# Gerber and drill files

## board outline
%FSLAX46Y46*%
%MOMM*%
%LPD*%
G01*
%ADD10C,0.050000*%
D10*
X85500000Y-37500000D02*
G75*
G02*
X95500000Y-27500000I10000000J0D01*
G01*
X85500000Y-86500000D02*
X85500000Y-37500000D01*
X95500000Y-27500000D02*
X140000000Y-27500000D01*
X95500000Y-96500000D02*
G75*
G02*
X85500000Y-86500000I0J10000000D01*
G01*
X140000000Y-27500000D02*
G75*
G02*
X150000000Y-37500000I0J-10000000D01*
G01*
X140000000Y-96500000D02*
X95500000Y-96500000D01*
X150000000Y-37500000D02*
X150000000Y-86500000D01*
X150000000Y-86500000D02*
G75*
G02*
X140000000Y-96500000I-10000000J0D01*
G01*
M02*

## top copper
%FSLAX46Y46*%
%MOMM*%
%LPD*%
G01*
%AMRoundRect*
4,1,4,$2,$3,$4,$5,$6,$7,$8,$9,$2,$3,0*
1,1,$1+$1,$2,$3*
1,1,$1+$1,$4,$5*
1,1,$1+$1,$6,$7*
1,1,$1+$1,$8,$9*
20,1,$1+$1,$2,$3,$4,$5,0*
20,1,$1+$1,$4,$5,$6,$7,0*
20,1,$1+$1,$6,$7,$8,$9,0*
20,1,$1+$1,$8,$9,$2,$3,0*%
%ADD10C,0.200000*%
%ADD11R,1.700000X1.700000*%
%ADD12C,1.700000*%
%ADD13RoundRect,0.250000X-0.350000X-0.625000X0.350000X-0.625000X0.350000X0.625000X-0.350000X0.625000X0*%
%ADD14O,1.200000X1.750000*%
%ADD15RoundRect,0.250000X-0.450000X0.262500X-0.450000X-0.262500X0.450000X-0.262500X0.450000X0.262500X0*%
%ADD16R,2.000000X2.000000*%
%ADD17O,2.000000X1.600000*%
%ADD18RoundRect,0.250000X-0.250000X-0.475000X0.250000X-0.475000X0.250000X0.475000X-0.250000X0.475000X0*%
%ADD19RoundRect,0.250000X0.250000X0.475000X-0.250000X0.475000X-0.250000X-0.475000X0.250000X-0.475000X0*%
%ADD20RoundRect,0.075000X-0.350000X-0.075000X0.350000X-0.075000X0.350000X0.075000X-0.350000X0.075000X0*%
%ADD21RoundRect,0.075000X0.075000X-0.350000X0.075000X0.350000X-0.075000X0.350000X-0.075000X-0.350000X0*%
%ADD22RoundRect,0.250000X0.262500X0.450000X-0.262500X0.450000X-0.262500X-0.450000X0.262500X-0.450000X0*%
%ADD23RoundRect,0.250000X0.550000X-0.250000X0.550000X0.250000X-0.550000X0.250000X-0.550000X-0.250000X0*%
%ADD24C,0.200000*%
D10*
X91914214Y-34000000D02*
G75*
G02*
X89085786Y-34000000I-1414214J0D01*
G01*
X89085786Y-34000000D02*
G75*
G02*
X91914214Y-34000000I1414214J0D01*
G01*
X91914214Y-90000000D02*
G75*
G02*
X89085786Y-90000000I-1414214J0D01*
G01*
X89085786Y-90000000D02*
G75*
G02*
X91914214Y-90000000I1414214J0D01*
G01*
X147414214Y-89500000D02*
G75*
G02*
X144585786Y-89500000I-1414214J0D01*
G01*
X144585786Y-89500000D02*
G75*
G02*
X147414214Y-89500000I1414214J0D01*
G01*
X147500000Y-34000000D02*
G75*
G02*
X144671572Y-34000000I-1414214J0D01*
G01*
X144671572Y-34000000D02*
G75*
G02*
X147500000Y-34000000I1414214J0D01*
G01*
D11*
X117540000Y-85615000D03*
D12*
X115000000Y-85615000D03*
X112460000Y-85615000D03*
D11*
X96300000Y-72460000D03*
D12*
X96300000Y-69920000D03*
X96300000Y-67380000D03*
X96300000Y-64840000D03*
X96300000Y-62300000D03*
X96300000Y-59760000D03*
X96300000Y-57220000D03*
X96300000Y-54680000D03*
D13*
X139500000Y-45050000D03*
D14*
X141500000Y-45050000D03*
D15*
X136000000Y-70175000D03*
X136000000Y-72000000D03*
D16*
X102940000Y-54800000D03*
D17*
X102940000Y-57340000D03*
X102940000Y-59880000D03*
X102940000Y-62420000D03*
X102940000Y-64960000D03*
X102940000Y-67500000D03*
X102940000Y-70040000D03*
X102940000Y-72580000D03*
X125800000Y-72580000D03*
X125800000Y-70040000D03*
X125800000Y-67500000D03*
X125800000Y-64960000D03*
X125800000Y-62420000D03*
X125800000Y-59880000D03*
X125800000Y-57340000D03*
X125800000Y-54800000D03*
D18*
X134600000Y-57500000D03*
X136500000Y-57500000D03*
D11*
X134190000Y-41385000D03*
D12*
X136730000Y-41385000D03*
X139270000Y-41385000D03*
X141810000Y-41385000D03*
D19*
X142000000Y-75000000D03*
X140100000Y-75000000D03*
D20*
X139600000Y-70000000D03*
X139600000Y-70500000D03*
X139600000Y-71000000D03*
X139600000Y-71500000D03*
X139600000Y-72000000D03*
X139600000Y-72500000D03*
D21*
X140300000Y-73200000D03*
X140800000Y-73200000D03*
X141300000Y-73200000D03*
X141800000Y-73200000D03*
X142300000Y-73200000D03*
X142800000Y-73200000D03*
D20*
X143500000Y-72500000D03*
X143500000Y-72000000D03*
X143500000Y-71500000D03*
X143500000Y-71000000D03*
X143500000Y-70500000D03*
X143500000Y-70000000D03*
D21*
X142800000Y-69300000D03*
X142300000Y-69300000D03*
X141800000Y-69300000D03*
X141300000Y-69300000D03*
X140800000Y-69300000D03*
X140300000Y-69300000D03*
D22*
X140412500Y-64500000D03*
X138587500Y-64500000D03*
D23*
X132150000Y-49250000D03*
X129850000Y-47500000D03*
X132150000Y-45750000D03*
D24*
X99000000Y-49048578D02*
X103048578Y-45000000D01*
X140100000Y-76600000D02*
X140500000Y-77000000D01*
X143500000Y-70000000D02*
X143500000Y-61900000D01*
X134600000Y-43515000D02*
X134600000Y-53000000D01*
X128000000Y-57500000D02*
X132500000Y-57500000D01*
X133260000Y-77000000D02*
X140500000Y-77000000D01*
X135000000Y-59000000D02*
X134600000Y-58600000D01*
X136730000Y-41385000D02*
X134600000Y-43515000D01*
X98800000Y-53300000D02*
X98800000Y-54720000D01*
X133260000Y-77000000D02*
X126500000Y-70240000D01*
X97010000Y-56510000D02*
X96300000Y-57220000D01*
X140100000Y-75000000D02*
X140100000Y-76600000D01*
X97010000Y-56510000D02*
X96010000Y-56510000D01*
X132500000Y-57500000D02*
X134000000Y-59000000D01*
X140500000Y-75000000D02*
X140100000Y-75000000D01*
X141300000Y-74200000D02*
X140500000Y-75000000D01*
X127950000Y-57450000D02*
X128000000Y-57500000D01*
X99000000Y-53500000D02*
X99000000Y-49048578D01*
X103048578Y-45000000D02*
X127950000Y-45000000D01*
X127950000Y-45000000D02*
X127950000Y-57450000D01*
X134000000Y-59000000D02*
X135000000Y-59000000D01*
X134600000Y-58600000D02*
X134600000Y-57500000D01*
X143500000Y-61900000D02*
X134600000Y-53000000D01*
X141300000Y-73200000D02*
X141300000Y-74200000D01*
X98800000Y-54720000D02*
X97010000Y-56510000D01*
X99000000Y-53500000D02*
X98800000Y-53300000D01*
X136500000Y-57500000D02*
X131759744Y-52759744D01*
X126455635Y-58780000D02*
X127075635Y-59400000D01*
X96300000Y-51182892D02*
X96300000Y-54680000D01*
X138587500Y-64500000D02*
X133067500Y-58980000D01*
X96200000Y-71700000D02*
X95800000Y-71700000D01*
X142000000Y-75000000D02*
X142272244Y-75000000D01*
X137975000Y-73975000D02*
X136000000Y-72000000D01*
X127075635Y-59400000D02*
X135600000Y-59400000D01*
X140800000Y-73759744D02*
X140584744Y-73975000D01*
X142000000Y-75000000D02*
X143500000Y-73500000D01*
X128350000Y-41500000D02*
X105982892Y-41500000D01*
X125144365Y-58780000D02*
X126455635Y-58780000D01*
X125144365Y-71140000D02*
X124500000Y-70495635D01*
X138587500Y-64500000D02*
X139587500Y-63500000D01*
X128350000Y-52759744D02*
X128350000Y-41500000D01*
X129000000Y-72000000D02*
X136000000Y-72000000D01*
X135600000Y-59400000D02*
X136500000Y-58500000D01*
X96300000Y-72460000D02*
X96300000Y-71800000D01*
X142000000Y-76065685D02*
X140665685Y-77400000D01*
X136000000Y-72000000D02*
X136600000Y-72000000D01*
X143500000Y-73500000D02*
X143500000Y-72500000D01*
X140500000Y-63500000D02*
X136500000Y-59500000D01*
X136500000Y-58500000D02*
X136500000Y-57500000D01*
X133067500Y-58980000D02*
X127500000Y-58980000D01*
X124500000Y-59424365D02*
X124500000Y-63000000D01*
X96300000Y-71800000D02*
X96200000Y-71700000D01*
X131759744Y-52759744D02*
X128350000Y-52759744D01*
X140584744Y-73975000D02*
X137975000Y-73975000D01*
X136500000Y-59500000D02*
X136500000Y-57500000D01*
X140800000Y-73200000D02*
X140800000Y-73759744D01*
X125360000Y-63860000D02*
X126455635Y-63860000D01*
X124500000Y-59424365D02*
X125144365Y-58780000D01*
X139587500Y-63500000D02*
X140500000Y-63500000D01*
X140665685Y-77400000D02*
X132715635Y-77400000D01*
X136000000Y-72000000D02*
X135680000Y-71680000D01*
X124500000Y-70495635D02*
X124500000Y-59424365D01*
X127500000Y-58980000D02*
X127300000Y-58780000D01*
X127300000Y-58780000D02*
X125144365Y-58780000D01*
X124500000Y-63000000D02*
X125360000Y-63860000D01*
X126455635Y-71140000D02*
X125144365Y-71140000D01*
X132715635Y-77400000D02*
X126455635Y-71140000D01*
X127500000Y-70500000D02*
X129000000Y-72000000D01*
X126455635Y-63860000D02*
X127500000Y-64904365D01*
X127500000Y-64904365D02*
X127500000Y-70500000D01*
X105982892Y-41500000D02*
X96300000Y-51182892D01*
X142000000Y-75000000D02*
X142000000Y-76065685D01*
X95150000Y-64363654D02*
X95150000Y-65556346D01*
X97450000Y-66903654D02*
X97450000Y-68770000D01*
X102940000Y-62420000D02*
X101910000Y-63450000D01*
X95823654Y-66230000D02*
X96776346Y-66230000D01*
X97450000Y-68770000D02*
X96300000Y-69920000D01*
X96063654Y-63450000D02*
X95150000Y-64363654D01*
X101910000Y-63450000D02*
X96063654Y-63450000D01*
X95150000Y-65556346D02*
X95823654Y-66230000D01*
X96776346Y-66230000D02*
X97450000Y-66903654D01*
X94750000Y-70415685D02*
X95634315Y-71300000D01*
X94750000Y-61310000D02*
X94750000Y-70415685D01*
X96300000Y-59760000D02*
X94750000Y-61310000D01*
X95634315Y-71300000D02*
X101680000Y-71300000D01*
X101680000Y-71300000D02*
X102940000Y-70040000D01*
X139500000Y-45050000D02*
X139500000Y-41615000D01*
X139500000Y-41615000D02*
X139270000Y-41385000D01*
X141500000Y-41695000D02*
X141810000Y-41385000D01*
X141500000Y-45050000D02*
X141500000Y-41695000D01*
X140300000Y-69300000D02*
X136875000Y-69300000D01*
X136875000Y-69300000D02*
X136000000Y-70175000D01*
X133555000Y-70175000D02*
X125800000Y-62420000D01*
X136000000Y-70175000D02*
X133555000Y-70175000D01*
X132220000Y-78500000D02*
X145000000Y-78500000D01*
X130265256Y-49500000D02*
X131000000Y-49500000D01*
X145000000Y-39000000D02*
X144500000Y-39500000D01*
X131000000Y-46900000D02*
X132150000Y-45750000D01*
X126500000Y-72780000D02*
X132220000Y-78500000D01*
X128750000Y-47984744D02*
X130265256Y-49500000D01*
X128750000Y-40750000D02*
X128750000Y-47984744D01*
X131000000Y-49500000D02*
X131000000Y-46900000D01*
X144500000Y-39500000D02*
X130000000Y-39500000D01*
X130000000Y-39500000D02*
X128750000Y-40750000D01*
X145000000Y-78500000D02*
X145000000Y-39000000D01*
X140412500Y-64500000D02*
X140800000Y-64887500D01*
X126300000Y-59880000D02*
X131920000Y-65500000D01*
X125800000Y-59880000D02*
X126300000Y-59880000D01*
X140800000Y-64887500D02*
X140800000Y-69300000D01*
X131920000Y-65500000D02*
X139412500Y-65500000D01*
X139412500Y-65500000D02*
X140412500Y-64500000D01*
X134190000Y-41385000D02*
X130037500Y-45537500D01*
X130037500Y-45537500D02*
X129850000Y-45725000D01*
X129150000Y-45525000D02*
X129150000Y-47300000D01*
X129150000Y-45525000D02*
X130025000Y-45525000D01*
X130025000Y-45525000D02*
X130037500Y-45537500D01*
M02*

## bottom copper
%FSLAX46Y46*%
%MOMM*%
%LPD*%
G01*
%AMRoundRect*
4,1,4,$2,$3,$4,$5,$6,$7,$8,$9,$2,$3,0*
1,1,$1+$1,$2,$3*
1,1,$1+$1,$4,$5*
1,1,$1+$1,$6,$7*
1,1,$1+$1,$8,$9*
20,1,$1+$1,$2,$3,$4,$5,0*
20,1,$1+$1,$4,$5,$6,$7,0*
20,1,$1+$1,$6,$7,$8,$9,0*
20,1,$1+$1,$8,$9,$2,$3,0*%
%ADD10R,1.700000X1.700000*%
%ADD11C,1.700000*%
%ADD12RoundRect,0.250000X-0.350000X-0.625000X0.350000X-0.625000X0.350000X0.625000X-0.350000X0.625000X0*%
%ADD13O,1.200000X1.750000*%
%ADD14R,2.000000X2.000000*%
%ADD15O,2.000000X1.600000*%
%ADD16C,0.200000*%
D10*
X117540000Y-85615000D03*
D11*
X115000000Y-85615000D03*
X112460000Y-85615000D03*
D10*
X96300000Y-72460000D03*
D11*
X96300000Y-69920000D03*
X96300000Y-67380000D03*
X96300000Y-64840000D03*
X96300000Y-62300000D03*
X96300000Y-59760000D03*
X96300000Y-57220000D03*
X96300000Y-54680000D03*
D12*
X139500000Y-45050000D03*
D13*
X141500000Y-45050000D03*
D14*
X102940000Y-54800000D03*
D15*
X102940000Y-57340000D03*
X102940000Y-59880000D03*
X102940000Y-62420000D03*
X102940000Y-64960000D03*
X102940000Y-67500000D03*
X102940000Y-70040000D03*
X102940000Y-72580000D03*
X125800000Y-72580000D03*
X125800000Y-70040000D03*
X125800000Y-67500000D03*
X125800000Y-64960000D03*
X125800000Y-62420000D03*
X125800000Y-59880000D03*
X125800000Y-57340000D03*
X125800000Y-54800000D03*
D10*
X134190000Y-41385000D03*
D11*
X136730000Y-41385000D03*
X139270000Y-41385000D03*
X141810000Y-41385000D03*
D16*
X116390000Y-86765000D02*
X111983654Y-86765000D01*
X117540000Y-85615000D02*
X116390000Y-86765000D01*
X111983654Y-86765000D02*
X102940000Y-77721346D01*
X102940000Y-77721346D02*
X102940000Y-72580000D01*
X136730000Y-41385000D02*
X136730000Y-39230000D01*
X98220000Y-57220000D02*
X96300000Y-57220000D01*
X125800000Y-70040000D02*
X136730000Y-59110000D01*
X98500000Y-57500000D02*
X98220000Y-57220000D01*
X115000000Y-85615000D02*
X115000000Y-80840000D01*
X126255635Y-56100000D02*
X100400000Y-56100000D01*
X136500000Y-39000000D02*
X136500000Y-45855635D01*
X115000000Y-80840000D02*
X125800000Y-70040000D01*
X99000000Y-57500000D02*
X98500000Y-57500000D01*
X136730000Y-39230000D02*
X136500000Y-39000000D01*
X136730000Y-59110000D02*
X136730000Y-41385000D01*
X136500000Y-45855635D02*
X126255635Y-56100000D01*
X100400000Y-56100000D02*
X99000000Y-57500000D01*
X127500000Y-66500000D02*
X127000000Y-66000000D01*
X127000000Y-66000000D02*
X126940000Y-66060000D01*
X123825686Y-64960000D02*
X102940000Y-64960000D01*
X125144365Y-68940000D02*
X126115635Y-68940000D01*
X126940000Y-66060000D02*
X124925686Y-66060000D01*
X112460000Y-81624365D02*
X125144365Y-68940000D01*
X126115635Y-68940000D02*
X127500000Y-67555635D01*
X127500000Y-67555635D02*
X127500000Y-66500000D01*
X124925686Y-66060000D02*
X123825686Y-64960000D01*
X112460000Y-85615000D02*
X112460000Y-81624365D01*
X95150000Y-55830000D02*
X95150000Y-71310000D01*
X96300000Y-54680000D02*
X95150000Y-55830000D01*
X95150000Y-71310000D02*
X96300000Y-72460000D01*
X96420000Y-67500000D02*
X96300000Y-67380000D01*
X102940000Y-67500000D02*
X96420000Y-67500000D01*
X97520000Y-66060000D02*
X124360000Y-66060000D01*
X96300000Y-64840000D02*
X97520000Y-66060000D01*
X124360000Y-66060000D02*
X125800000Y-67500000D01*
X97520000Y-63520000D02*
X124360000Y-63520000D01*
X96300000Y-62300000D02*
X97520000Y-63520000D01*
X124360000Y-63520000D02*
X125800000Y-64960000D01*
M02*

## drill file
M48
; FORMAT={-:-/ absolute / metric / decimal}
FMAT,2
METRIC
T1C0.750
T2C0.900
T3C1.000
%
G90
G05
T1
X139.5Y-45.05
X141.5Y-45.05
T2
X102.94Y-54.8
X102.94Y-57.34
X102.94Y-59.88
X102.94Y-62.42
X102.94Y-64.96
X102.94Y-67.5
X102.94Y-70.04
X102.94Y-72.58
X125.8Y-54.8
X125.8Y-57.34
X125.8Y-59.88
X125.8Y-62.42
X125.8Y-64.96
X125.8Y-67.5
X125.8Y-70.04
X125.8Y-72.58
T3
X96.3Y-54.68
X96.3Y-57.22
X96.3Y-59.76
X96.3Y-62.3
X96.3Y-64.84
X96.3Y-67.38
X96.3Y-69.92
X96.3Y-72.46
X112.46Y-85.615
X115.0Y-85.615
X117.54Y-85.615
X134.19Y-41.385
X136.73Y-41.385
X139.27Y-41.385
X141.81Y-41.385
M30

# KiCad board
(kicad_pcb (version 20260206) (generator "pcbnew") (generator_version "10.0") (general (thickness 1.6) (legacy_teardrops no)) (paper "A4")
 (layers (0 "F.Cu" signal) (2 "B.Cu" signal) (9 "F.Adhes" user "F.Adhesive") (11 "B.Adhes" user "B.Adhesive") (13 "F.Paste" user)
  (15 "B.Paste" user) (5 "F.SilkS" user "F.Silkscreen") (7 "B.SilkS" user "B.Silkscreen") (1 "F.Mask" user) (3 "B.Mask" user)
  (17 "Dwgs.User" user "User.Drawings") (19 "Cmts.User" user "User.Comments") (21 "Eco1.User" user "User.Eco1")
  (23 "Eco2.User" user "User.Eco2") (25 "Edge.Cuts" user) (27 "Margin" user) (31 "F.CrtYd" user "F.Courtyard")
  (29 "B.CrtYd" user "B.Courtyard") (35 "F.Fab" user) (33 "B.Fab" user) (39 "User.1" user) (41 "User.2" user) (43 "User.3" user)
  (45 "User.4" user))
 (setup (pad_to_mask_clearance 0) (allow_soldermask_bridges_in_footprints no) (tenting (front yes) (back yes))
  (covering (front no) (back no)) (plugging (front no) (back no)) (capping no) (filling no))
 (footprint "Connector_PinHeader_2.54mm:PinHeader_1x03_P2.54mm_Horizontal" (layer "F.Cu") (at 117.54 85.615 -90)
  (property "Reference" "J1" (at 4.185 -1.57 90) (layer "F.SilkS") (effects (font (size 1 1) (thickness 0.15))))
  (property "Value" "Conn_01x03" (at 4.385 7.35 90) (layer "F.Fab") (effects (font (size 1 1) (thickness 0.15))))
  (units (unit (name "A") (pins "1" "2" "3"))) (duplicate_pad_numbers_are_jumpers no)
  (pad "1" thru_hole rect (at 0 0 270) (size 1.7 1.7) (drill 1) (layers "*.Cu" "*.Mask") (remove_unused_layers no) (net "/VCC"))
  (pad "2" thru_hole circle (at 0 2.54 270) (size 1.7 1.7) (drill 1) (layers "*.Cu" "*.Mask") (remove_unused_layers no) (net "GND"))
  (pad "3" thru_hole circle (at 0 5.08 270) (size 1.7 1.7) (drill 1) (layers "*.Cu" "*.Mask") (remove_unused_layers no) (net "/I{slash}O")))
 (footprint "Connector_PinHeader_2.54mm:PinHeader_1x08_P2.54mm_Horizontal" (layer "F.Cu") (at 96.3 72.46 180)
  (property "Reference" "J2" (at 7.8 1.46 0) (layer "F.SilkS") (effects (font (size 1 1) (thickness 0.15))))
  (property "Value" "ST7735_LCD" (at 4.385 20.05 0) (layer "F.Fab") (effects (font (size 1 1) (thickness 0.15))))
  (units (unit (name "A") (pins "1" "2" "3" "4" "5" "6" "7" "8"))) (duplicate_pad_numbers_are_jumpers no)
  (pad "1" thru_hole rect (at 0 0 180) (size 1.7 1.7) (drill 1) (layers "*.Cu" "*.Mask") (remove_unused_layers no) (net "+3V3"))
  (pad "2" thru_hole circle (at 0 2.54 180) (size 1.7 1.7) (drill 1) (layers "*.Cu" "*.Mask") (remove_unused_layers no) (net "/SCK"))
  (pad "3" thru_hole circle (at 0 5.08 180) (size 1.7 1.7) (drill 1) (layers "*.Cu" "*.Mask") (remove_unused_layers no) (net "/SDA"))
  (pad "4" thru_hole circle (at 0 7.62 180) (size 1.7 1.7) (drill 1) (layers "*.Cu" "*.Mask") (remove_unused_layers no) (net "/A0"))
  (pad "5" thru_hole circle (at 0 10.16 180) (size 1.7 1.7) (drill 1) (layers "*.Cu" "*.Mask") (remove_unused_layers no) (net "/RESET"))
  (pad "6" thru_hole circle (at 0 12.7 180) (size 1.7 1.7) (drill 1) (layers "*.Cu" "*.Mask") (remove_unused_layers no) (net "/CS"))
  (pad "7" thru_hole circle (at 0 15.24 180) (size 1.7 1.7) (drill 1) (layers "*.Cu" "*.Mask") (remove_unused_layers no) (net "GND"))
  (pad "8" thru_hole circle (at 0 17.78 180) (size 1.7 1.7) (drill 1) (layers "*.Cu" "*.Mask") (remove_unused_layers no) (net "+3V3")))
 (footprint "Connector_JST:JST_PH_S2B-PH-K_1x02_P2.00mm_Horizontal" (layer "F.Cu") (at 139.5 45.05)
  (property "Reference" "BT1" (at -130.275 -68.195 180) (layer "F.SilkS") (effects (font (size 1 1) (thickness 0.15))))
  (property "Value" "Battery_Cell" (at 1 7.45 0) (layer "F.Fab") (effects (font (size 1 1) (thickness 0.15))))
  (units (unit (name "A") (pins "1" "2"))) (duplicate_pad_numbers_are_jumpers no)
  (pad "1" thru_hole roundrect (at 0 0) (size 1.2 1.75) (drill 0.75) (layers "*.Cu" "*.Mask") (remove_unused_layers no)
   (roundrect_rratio 0.208333) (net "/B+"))
  (pad "2" thru_hole oval (at 2 0) (size 1.2 1.75) (drill 0.75) (layers "*.Cu" "*.Mask") (remove_unused_layers no) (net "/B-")))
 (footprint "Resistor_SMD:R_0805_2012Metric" (layer "F.Cu") (at 136 71.0875 -90)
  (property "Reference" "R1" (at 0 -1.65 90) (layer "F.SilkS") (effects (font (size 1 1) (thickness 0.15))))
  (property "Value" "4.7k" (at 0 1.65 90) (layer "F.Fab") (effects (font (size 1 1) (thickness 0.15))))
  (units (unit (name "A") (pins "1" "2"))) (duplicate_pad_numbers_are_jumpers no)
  (pad "1" smd roundrect (at -0.9125 0 270) (size 1.025 1.4) (layers "F.Cu" "F.Mask" "F.Paste") (roundrect_rratio 0.243902)
   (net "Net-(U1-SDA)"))
  (pad "2" smd roundrect (at 0.9125 0 270) (size 1.025 1.4) (layers "F.Cu" "F.Mask" "F.Paste") (roundrect_rratio 0.243902) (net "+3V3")))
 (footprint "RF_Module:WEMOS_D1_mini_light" (layer "F.Cu") (at 102.94 54.8)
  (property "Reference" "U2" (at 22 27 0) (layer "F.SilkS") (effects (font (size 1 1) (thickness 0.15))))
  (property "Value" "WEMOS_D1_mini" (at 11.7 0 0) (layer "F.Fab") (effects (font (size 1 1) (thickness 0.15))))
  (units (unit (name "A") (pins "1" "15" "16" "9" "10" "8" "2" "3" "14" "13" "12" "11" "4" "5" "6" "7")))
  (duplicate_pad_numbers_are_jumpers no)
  (pad "1" thru_hole rect (at 0 0) (size 2 2) (drill 0.9) (layers "*.Cu" "*.Mask") (remove_unused_layers no)
   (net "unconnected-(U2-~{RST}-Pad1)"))
  (pad "2" thru_hole oval (at 0 2.54) (size 2 1.6) (drill 0.9) (layers "*.Cu" "*.Mask") (remove_unused_layers no)
   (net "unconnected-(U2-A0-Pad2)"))
  (pad "3" thru_hole oval (at 0 5.08) (size 2 1.6) (drill 0.9) (layers "*.Cu" "*.Mask") (remove_unused_layers no)
   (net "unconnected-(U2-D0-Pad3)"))
  (pad "4" thru_hole oval (at 0 7.62) (size 2 1.6) (drill 0.9) (layers "*.Cu" "*.Mask") (remove_unused_layers no) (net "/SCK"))
  (pad "5" thru_hole oval (at 0 10.16) (size 2 1.6) (drill 0.9) (layers "*.Cu" "*.Mask") (remove_unused_layers no) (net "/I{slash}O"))
  (pad "6" thru_hole oval (at 0 12.7) (size 2 1.6) (drill 0.9) (layers "*.Cu" "*.Mask") (remove_unused_layers no) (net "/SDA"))
  (pad "7" thru_hole oval (at 0 15.24) (size 2 1.6) (drill 0.9) (layers "*.Cu" "*.Mask") (remove_unused_layers no) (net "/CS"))
  (pad "8" thru_hole oval (at 0 17.78) (size 2 1.6) (drill 0.9) (layers "*.Cu" "*.Mask") (remove_unused_layers no) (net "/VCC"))
  (pad "9" thru_hole oval (at 22.86 17.78) (size 2 1.6) (drill 0.9) (layers "*.Cu" "*.Mask") (remove_unused_layers no) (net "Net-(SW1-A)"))
  (pad "10" thru_hole oval (at 22.86 15.24) (size 2 1.6) (drill 0.9) (layers "*.Cu" "*.Mask") (remove_unused_layers no) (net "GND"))
  (pad "11" thru_hole oval (at 22.86 12.7) (size 2 1.6) (drill 0.9) (layers "*.Cu" "*.Mask") (remove_unused_layers no) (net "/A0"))
  (pad "12" thru_hole oval (at 22.86 10.16) (size 2 1.6) (drill 0.9) (layers "*.Cu" "*.Mask") (remove_unused_layers no) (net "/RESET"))
  (pad "13" thru_hole oval (at 22.86 7.62) (size 2 1.6) (drill 0.9) (layers "*.Cu" "*.Mask") (remove_unused_layers no) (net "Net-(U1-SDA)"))
  (pad "14" thru_hole oval (at 22.86 5.08) (size 2 1.6) (drill 0.9) (layers "*.Cu" "*.Mask") (remove_unused_layers no) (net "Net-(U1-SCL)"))
  (pad "15" thru_hole oval (at 22.86 2.54) (size 2 1.6) (drill 0.9) (layers "*.Cu" "*.Mask") (remove_unused_layers no)
   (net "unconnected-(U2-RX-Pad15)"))
  (pad "16" thru_hole oval (at 22.86 0) (size 2 1.6) (drill 0.9) (layers "*.Cu" "*.Mask") (remove_unused_layers no)
   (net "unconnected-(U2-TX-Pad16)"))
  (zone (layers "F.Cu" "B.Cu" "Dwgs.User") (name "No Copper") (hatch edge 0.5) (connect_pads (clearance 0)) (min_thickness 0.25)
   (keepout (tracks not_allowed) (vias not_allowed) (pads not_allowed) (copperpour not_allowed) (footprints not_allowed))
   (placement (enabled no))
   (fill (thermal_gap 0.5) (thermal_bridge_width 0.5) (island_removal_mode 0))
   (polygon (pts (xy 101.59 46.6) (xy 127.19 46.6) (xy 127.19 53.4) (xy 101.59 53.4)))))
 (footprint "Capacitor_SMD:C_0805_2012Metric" (layer "F.Cu") (at 135.55 57.5)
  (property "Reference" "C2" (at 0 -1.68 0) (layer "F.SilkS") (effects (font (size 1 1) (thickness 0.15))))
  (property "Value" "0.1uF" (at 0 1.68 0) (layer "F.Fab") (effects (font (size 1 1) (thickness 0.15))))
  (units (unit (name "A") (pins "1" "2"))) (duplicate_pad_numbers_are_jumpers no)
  (pad "1" smd roundrect (at -0.95 0) (size 1 1.45) (layers "F.Cu" "F.Mask" "F.Paste") (roundrect_rratio 0.25) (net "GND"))
  (pad "2" smd roundrect (at 0.95 0) (size 1 1.45) (layers "F.Cu" "F.Mask" "F.Paste") (roundrect_rratio 0.25) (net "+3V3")))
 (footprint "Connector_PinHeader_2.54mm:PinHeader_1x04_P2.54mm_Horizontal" (layer "F.Cu") (at 134.19 41.385 90)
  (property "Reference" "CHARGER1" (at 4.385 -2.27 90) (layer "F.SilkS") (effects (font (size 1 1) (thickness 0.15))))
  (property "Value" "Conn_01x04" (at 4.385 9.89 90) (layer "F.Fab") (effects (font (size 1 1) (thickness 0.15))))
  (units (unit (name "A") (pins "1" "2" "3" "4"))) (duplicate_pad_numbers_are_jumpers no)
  (pad "1" thru_hole rect (at 0 0 90) (size 1.7 1.7) (drill 1) (layers "*.Cu" "*.Mask") (remove_unused_layers no) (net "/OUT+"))
  (pad "2" thru_hole circle (at 0 2.54 90) (size 1.7 1.7) (drill 1) (layers "*.Cu" "*.Mask") (remove_unused_layers no) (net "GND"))
  (pad "3" thru_hole circle (at 0 5.08 90) (size 1.7 1.7) (drill 1) (layers "*.Cu" "*.Mask") (remove_unused_layers no) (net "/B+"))
  (pad "4" thru_hole circle (at 0 7.62 90) (size 1.7 1.7) (drill 1) (layers "*.Cu" "*.Mask") (remove_unused_layers no) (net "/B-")))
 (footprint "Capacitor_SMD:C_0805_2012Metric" (layer "F.Cu") (at 141.05 75 180)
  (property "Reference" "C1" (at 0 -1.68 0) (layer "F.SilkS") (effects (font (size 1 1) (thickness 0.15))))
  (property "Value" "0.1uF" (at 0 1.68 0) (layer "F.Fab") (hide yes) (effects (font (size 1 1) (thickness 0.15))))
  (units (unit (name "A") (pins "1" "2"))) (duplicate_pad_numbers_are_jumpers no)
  (pad "1" smd roundrect (at -0.95 0 180) (size 1 1.45) (layers "F.Cu" "F.Mask" "F.Paste") (roundrect_rratio 0.25) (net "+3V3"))
  (pad "2" smd roundrect (at 0.95 0 180) (size 1 1.45) (layers "F.Cu" "F.Mask" "F.Paste") (roundrect_rratio 0.25) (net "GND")))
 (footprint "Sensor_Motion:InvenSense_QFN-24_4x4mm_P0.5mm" (layer "F.Cu") (at 141.55 71.25)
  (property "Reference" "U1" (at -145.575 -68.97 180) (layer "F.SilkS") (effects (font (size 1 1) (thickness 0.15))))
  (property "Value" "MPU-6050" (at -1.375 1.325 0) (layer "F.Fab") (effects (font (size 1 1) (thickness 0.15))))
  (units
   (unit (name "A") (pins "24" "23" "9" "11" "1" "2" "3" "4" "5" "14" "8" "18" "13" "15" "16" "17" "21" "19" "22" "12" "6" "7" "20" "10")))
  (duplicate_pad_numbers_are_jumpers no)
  (pad "1" smd roundrect (at -1.95 -1.25) (size 0.85 0.3) (layers "F.Cu" "F.Mask" "F.Paste") (roundrect_rratio 0.25)
   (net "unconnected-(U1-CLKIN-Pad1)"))
  (pad "2" smd roundrect (at -1.95 -0.75) (size 0.85 0.3) (layers "F.Cu" "F.Mask" "F.Paste") (roundrect_rratio 0.25)
   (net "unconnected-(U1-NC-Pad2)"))
  (pad "3" smd roundrect (at -1.95 -0.25) (size 0.85 0.3) (layers "F.Cu" "F.Mask" "F.Paste") (roundrect_rratio 0.25)
   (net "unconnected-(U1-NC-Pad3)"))
  (pad "4" smd roundrect (at -1.95 0.25) (size 0.85 0.3) (layers "F.Cu" "F.Mask" "F.Paste") (roundrect_rratio 0.25)
   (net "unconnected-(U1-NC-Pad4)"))
  (pad "5" smd roundrect (at -1.95 0.75) (size 0.85 0.3) (layers "F.Cu" "F.Mask" "F.Paste") (roundrect_rratio 0.25)
   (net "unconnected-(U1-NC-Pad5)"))
  (pad "6" smd roundrect (at -1.95 1.25) (size 0.85 0.3) (layers "F.Cu" "F.Mask" "F.Paste") (roundrect_rratio 0.25)
   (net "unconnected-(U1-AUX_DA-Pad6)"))
  (pad "7" smd roundrect (at -1.25 1.95 90) (size 0.85 0.3) (layers "F.Cu" "F.Mask" "F.Paste") (roundrect_rratio 0.25)
   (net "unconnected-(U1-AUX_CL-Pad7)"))
  (pad "8" smd roundrect (at -0.75 1.95 90) (size 0.85 0.3) (layers "F.Cu" "F.Mask" "F.Paste") (roundrect_rratio 0.25) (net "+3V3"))
  (pad "9" smd roundrect (at -0.25 1.95 90) (size 0.85 0.3) (layers "F.Cu" "F.Mask" "F.Paste") (roundrect_rratio 0.25) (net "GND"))
  (pad "10" smd roundrect (at 0.25 1.95 90) (size 0.85 0.3) (layers "F.Cu" "F.Mask" "F.Paste") (roundrect_rratio 0.25)
   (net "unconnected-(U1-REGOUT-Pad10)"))
  (pad "11" smd roundrect (at 0.75 1.95 90) (size 0.85 0.3) (layers "F.Cu" "F.Mask" "F.Paste") (roundrect_rratio 0.25)
   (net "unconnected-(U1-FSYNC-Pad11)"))
  (pad "12" smd roundrect (at 1.25 1.95 90) (size 0.85 0.3) (layers "F.Cu" "F.Mask" "F.Paste") (roundrect_rratio 0.25)
   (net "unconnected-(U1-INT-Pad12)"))
  (pad "13" smd roundrect (at 1.95 1.25) (size 0.85 0.3) (layers "F.Cu" "F.Mask" "F.Paste") (roundrect_rratio 0.25) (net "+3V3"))
  (pad "14" smd roundrect (at 1.95 0.75) (size 0.85 0.3) (layers "F.Cu" "F.Mask" "F.Paste") (roundrect_rratio 0.25)
   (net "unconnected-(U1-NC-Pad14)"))
  (pad "15" smd roundrect (at 1.95 0.25) (size 0.85 0.3) (layers "F.Cu" "F.Mask" "F.Paste") (roundrect_rratio 0.25)
   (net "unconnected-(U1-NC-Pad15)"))
  (pad "16" smd roundrect (at 1.95 -0.25) (size 0.85 0.3) (layers "F.Cu" "F.Mask" "F.Paste") (roundrect_rratio 0.25)
   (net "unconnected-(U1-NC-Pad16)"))
  (pad "17" smd roundrect (at 1.95 -0.75) (size 0.85 0.3) (layers "F.Cu" "F.Mask" "F.Paste") (roundrect_rratio 0.25)
   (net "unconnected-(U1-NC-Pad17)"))
  (pad "18" smd roundrect (at 1.95 -1.25) (size 0.85 0.3) (layers "F.Cu" "F.Mask" "F.Paste") (roundrect_rratio 0.25) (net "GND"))
  (pad "19" smd roundrect (at 1.25 -1.95 90) (size 0.85 0.3) (layers "F.Cu" "F.Mask" "F.Paste") (roundrect_rratio 0.25)
   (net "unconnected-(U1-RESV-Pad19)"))
  (pad "20" smd roundrect (at 0.75 -1.95 90) (size 0.85 0.3) (layers "F.Cu" "F.Mask" "F.Paste") (roundrect_rratio 0.25)
   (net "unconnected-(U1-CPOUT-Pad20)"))
  (pad "21" smd roundrect (at 0.25 -1.95 90) (size 0.85 0.3) (layers "F.Cu" "F.Mask" "F.Paste") (roundrect_rratio 0.25)
   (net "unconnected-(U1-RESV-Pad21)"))
  (pad "22" smd roundrect (at -0.25 -1.95 90) (size 0.85 0.3) (layers "F.Cu" "F.Mask" "F.Paste") (roundrect_rratio 0.25)
   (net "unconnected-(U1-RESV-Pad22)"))
  (pad "23" smd roundrect (at -0.75 -1.95 90) (size 0.85 0.3) (layers "F.Cu" "F.Mask" "F.Paste") (roundrect_rratio 0.25)
   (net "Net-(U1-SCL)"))
  (pad "24" smd roundrect (at -1.25 -1.95 90) (size 0.85 0.3) (layers "F.Cu" "F.Mask" "F.Paste") (roundrect_rratio 0.25)
   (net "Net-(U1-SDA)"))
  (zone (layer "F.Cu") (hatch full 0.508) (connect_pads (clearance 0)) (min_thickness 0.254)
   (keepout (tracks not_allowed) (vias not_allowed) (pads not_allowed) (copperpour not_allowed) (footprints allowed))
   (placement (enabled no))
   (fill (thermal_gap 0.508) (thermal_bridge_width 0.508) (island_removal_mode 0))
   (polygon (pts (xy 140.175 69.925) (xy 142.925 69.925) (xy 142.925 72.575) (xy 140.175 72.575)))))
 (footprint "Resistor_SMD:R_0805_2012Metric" (layer "F.Cu") (at 139.5 64.5 180)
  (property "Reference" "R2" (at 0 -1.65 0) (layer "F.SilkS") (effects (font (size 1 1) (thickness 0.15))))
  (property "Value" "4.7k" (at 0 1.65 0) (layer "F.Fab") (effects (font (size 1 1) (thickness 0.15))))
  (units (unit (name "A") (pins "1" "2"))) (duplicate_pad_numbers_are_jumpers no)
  (pad "1" smd roundrect (at -0.9125 0 180) (size 1.025 1.4) (layers "F.Cu" "F.Mask" "F.Paste") (roundrect_rratio 0.243902)
   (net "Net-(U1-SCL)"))
  (pad "2" smd roundrect (at 0.9125 0 180) (size 1.025 1.4) (layers "F.Cu" "F.Mask" "F.Paste") (roundrect_rratio 0.243902) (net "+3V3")))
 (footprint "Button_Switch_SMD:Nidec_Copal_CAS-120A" (layer "F.Cu") (at 131 47.5 180)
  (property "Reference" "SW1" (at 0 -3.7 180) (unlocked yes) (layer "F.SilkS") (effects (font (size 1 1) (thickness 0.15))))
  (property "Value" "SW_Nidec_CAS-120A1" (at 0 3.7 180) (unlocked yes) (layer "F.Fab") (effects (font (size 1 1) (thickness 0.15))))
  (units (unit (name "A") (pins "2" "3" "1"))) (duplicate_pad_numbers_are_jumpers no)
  (pad "1" smd roundrect (at -1.15 -1.75 90) (size 1 1.6) (layers "F.Cu" "F.Mask" "F.Paste") (roundrect_rratio 0.25)
   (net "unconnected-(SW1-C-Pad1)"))
  (pad "2" smd roundrect (at 1.15 0 90) (size 1 1.6) (layers "F.Cu" "F.Mask" "F.Paste") (roundrect_rratio 0.25) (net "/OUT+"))
  (pad "3" smd roundrect (at -1.15 1.75 90) (size 1 1.6) (layers "F.Cu" "F.Mask" "F.Paste") (roundrect_rratio 0.25) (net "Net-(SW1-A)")))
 (gr_circle (center 90.5 34) (end 91.5 35) (stroke (width 0.2) (type default)) (fill no) (layer "F.Cu"))
 (gr_circle (center 90.5 90) (end 91.5 91) (stroke (width 0.2) (type default)) (fill no) (layer "F.Cu"))
 (gr_circle (center 146 89.5) (end 147 90.5) (stroke (width 0.2) (type default)) (fill no) (layer "F.Cu"))
 (gr_circle (center 146.085786 34) (end 147.085786 35) (stroke (width 0.2) (type default)) (fill no) (layer "F.Cu"))
 (gr_arc (start 85.5 37.5) (mid 88.428932 30.428932) (end 95.5 27.5) (stroke (width 0.05) (type default)) (layer "Edge.Cuts"))
 (gr_line (start 85.5 86.5) (end 85.5 37.5) (stroke (width 0.05) (type default)) (layer "Edge.Cuts"))
 (gr_line (start 95.5 27.5) (end 140 27.5) (stroke (width 0.05) (type default)) (layer "Edge.Cuts"))
 (gr_arc (start 95.5 96.5) (mid 88.428932 93.571068) (end 85.5 86.5) (stroke (width 0.05) (type default)) (layer "Edge.Cuts"))
 (gr_arc (start 140 27.5) (mid 147.071068 30.428932) (end 150 37.5) (stroke (width 0.05) (type default)) (layer "Edge.Cuts"))
 (gr_line (start 140 96.5) (end 95.5 96.5) (stroke (width 0.05) (type default)) (layer "Edge.Cuts"))
 (gr_line (start 150 37.5) (end 150 86.5) (stroke (width 0.05) (type default)) (layer "Edge.Cuts"))
 (gr_arc (start 150 86.5) (mid 147.071068 93.571068) (end 140 96.5) (stroke (width 0.05) (type default)) (layer "Edge.Cuts"))
 (segment (start 116.39 86.765) (end 111.983654 86.765) (width 0.2) (layer "B.Cu") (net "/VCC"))
 (segment (start 117.54 85.615) (end 116.39 86.765) (width 0.2) (layer "B.Cu") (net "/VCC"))
 (segment (start 111.983654 86.765) (end 102.94 77.721346) (width 0.2) (layer "B.Cu") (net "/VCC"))
 (segment (start 102.94 77.721346) (end 102.94 72.58) (width 0.2) (layer "B.Cu") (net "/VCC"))
 (segment (start 99 49.048578) (end 103.048578 45) (width 0.2) (layer "F.Cu") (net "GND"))
 (segment (start 140.1 76.6) (end 140.5 77) (width 0.2) (layer "F.Cu") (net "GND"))
 (segment (start 143.5 70) (end 143.5 61.9) (width 0.2) (layer "F.Cu") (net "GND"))
 (segment (start 134.6 43.515) (end 134.6 53) (width 0.2) (layer "F.Cu") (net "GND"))
 (segment (start 128 57.5) (end 132.5 57.5) (width 0.2) (layer "F.Cu") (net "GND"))
 (segment (start 133.26 77) (end 140.5 77) (width 0.2) (layer "F.Cu") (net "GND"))
 (segment (start 135 59) (end 134.6 58.6) (width 0.2) (layer "F.Cu") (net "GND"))
 (segment (start 136.73 41.385) (end 134.6 43.515) (width 0.2) (layer "F.Cu") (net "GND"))
 (segment (start 98.8 53.3) (end 98.8 54.72) (width 0.2) (layer "F.Cu") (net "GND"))
 (segment (start 133.26 77) (end 126.5 70.24) (width 0.2) (layer "F.Cu") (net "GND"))
 (segment (start 97.01 56.51) (end 96.3 57.22) (width 0.2) (layer "F.Cu") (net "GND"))
 (segment (start 140.1 75) (end 140.1 76.6) (width 0.2) (layer "F.Cu") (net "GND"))
 (segment (start 97.01 56.51) (end 96.01 56.51) (width 0.2) (layer "F.Cu") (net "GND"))
 (segment (start 132.5 57.5) (end 134 59) (width 0.2) (layer "F.Cu") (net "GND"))
 (segment (start 140.5 75) (end 140.1 75) (width 0.2) (layer "F.Cu") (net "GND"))
 (segment (start 141.3 74.2) (end 140.5 75) (width 0.2) (layer "F.Cu") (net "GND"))
 (segment (start 127.95 57.45) (end 128 57.5) (width 0.2) (layer "F.Cu") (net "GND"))
 (segment (start 99 53.5) (end 99 49.048578) (width 0.2) (layer "F.Cu") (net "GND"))
 (segment (start 103.048578 45) (end 127.95 45) (width 0.2) (layer "F.Cu") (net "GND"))
 (segment (start 127.95 45) (end 127.95 57.45) (width 0.2) (layer "F.Cu") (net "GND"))
 (segment (start 134 59) (end 135 59) (width 0.2) (layer "F.Cu") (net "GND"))
 (segment (start 134.6 58.6) (end 134.6 57.5) (width 0.2) (layer "F.Cu") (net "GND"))
 (segment (start 143.5 61.9) (end 134.6 53) (width 0.2) (layer "F.Cu") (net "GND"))
 (segment (start 141.3 73.2) (end 141.3 74.2) (width 0.2) (layer "F.Cu") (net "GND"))
 (segment (start 98.8 54.72) (end 97.01 56.51) (width 0.2) (layer "F.Cu") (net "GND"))
 (segment (start 99 53.5) (end 98.8 53.3) (width 0.2) (layer "F.Cu") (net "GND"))
 (segment (start 136.73 41.385) (end 136.73 39.23) (width 0.2) (layer "B.Cu") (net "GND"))
 (segment (start 98.22 57.22) (end 96.3 57.22) (width 0.2) (layer "B.Cu") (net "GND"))
 (segment (start 125.8 70.04) (end 136.73 59.11) (width 0.2) (layer "B.Cu") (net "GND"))
 (segment (start 98.5 57.5) (end 98.22 57.22) (width 0.2) (layer "B.Cu") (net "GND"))
 (segment (start 115 85.615) (end 115 80.84) (width 0.2) (layer "B.Cu") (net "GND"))
 (segment (start 126.255635 56.1) (end 100.4 56.1) (width 0.2) (layer "B.Cu") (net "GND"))
 (segment (start 136.5 39) (end 136.5 45.855635) (width 0.2) (layer "B.Cu") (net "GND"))
 (segment (start 115 80.84) (end 125.8 70.04) (width 0.2) (layer "B.Cu") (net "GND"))
 (segment (start 99 57.5) (end 98.5 57.5) (width 0.2) (layer "B.Cu") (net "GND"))
 (segment (start 136.73 39.23) (end 136.5 39) (width 0.2) (layer "B.Cu") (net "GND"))
 (segment (start 136.73 59.11) (end 136.73 41.385) (width 0.2) (layer "B.Cu") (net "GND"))
 (segment (start 136.5 45.855635) (end 126.255635 56.1) (width 0.2) (layer "B.Cu") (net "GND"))
 (segment (start 100.4 56.1) (end 99 57.5) (width 0.2) (layer "B.Cu") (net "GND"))
 (segment (start 127.5 66.5) (end 127 66) (width 0.2) (layer "B.Cu") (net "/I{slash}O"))
 (segment (start 127 66) (end 126.94 66.06) (width 0.2) (layer "B.Cu") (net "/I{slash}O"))
 (segment (start 123.825686 64.96) (end 102.94 64.96) (width 0.2) (layer "B.Cu") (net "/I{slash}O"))
 (segment (start 125.144365 68.94) (end 126.115635 68.94) (width 0.2) (layer "B.Cu") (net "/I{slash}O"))
 (segment (start 126.94 66.06) (end 124.925686 66.06) (width 0.2) (layer "B.Cu") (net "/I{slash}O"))
 (segment (start 112.46 81.624365) (end 125.144365 68.94) (width 0.2) (layer "B.Cu") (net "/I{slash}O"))
 (segment (start 126.115635 68.94) (end 127.5 67.555635) (width 0.2) (layer "B.Cu") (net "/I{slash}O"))
 (segment (start 127.5 67.555635) (end 127.5 66.5) (width 0.2) (layer "B.Cu") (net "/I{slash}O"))
 (segment (start 124.925686 66.06) (end 123.825686 64.96) (width 0.2) (layer "B.Cu") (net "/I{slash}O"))
 (segment (start 112.46 85.615) (end 112.46 81.624365) (width 0.2) (layer "B.Cu") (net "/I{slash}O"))
 (segment (start 136.5 57.5) (end 131.759744 52.759744) (width 0.2) (layer "F.Cu") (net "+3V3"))
 (segment (start 126.455635 58.78) (end 127.075635 59.4) (width 0.2) (layer "F.Cu") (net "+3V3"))
 (segment (start 96.3 51.182892) (end 96.3 54.68) (width 0.2) (layer "F.Cu") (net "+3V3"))
 (segment (start 138.5875 64.5) (end 133.0675 58.98) (width 0.2) (layer "F.Cu") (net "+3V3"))
 (segment (start 96.2 71.7) (end 95.8 71.7) (width 0.2) (layer "F.Cu") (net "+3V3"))
 (segment (start 142 75) (end 142.272244 75) (width 0.2) (layer "F.Cu") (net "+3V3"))
 (segment (start 137.975 73.975) (end 136 72) (width 0.2) (layer "F.Cu") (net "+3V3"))
 (segment (start 127.075635 59.4) (end 135.6 59.4) (width 0.2) (layer "F.Cu") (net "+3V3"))
 (segment (start 140.8 73.759744) (end 140.584744 73.975) (width 0.2) (layer "F.Cu") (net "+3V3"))
 (segment (start 142 75) (end 143.5 73.5) (width 0.2) (layer "F.Cu") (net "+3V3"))
 (segment (start 128.35 41.5) (end 105.982892 41.5) (width 0.2) (layer "F.Cu") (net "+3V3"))
 (segment (start 125.144365 58.78) (end 126.455635 58.78) (width 0.2) (layer "F.Cu") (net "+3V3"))
 (segment (start 125.144365 71.14) (end 124.5 70.495635) (width 0.2) (layer "F.Cu") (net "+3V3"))
 (segment (start 138.5875 64.5) (end 139.5875 63.5) (width 0.2) (layer "F.Cu") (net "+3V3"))
 (segment (start 128.35 52.759744) (end 128.35 41.5) (width 0.2) (layer "F.Cu") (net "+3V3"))
 (segment (start 129 72) (end 136 72) (width 0.2) (layer "F.Cu") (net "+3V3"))
 (segment (start 135.6 59.4) (end 136.5 58.5) (width 0.2) (layer "F.Cu") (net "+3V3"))
 (segment (start 96.3 72.46) (end 96.3 71.8) (width 0.2) (layer "F.Cu") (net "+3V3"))
 (segment (start 142 76.065685) (end 140.665685 77.4) (width 0.2) (layer "F.Cu") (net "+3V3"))
 (segment (start 136 72) (end 136.6 72) (width 0.2) (layer "F.Cu") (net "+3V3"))
 (segment (start 143.5 73.5) (end 143.5 72.5) (width 0.2) (layer "F.Cu") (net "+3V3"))
 (segment (start 140.5 63.5) (end 136.5 59.5) (width 0.2) (layer "F.Cu") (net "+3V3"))
 (segment (start 136.5 58.5) (end 136.5 57.5) (width 0.2) (layer "F.Cu") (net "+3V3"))
 (segment (start 133.0675 58.98) (end 127.5 58.98) (width 0.2) (layer "F.Cu") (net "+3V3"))
 (segment (start 124.5 59.424365) (end 124.5 63) (width 0.2) (layer "F.Cu") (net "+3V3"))
 (segment (start 96.3 71.8) (end 96.2 71.7) (width 0.2) (layer "F.Cu") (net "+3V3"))
 (segment (start 131.759744 52.759744) (end 128.35 52.759744) (width 0.2) (layer "F.Cu") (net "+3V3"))
 (segment (start 140.584744 73.975) (end 137.975 73.975) (width 0.2) (layer "F.Cu") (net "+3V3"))
 (segment (start 136.5 59.5) (end 136.5 57.5) (width 0.2) (layer "F.Cu") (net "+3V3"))
 (segment (start 140.8 73.2) (end 140.8 73.759744) (width 0.2) (layer "F.Cu") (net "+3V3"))
 (segment (start 125.36 63.86) (end 126.455635 63.86) (width 0.2) (layer "F.Cu") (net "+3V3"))
 (segment (start 124.5 59.424365) (end 125.144365 58.78) (width 0.2) (layer "F.Cu") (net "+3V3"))
 (segment (start 139.5875 63.5) (end 140.5 63.5) (width 0.2) (layer "F.Cu") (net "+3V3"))
 (segment (start 140.665685 77.4) (end 132.715635 77.4) (width 0.2) (layer "F.Cu") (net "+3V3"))
 (segment (start 136 72) (end 135.68 71.68) (width 0.2) (layer "F.Cu") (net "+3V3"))
 (segment (start 124.5 70.495635) (end 124.5 59.424365) (width 0.2) (layer "F.Cu") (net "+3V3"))
 (segment (start 127.5 58.98) (end 127.3 58.78) (width 0.2) (layer "F.Cu") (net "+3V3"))
 (segment (start 127.3 58.78) (end 125.144365 58.78) (width 0.2) (layer "F.Cu") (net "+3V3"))
 (segment (start 124.5 63) (end 125.36 63.86) (width 0.2) (layer "F.Cu") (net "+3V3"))
 (segment (start 126.455635 71.14) (end 125.144365 71.14) (width 0.2) (layer "F.Cu") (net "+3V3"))
 (segment (start 132.715635 77.4) (end 126.455635 71.14) (width 0.2) (layer "F.Cu") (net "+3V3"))
 (segment (start 127.5 70.5) (end 129 72) (width 0.2) (layer "F.Cu") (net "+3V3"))
 (segment (start 126.455635 63.86) (end 127.5 64.904365) (width 0.2) (layer "F.Cu") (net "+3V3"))
 (segment (start 127.5 64.904365) (end 127.5 70.5) (width 0.2) (layer "F.Cu") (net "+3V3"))
 (segment (start 105.982892 41.5) (end 96.3 51.182892) (width 0.2) (layer "F.Cu") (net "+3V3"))
 (segment (start 142 75) (end 142 76.065685) (width 0.2) (layer "F.Cu") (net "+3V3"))
 (segment (start 95.15 55.83) (end 95.15 71.31) (width 0.2) (layer "B.Cu") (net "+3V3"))
 (segment (start 96.3 54.68) (end 95.15 55.83) (width 0.2) (layer "B.Cu") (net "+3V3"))
 (segment (start 95.15 71.31) (end 96.3 72.46) (width 0.2) (layer "B.Cu") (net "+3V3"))
 (segment (start 95.15 64.363654) (end 95.15 65.556346) (width 0.2) (layer "F.Cu") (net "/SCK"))
 (segment (start 97.45 66.903654) (end 97.45 68.77) (width 0.2) (layer "F.Cu") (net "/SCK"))
 (segment (start 102.94 62.42) (end 101.91 63.45) (width 0.2) (layer "F.Cu") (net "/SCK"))
 (segment (start 95.823654 66.23) (end 96.776346 66.23) (width 0.2) (layer "F.Cu") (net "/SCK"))
 (segment (start 97.45 68.77) (end 96.3 69.92) (width 0.2) (layer "F.Cu") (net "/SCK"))
 (segment (start 96.063654 63.45) (end 95.15 64.363654) (width 0.2) (layer "F.Cu") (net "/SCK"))
 (segment (start 101.91 63.45) (end 96.063654 63.45) (width 0.2) (layer "F.Cu") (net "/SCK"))
 (segment (start 95.15 65.556346) (end 95.823654 66.23) (width 0.2) (layer "F.Cu") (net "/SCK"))
 (segment (start 96.776346 66.23) (end 97.45 66.903654) (width 0.2) (layer "F.Cu") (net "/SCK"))
 (segment (start 96.42 67.5) (end 96.3 67.38) (width 0.2) (layer "B.Cu") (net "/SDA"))
 (segment (start 102.94 67.5) (end 96.42 67.5) (width 0.2) (layer "B.Cu") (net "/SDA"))
 (segment (start 97.52 66.06) (end 124.36 66.06) (width 0.2) (layer "B.Cu") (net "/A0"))
 (segment (start 96.3 64.84) (end 97.52 66.06) (width 0.2) (layer "B.Cu") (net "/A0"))
 (segment (start 124.36 66.06) (end 125.8 67.5) (width 0.2) (layer "B.Cu") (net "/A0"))
 (segment (start 97.52 63.52) (end 124.36 63.52) (width 0.2) (layer "B.Cu") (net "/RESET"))
 (segment (start 96.3 62.3) (end 97.52 63.52) (width 0.2) (layer "B.Cu") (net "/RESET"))
 (segment (start 124.36 63.52) (end 125.8 64.96) (width 0.2) (layer "B.Cu") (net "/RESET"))
 (segment (start 94.75 70.415685) (end 95.634315 71.3) (width 0.2) (layer "F.Cu") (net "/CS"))
 (segment (start 94.75 61.31) (end 94.75 70.415685) (width 0.2) (layer "F.Cu") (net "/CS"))
 (segment (start 96.3 59.76) (end 94.75 61.31) (width 0.2) (layer "F.Cu") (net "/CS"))
 (segment (start 95.634315 71.3) (end 101.68 71.3) (width 0.2) (layer "F.Cu") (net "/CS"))
 (segment (start 101.68 71.3) (end 102.94 70.04) (width 0.2) (layer "F.Cu") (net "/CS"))
 (segment (start 139.5 45.05) (end 139.5 41.615) (width 0.2) (layer "F.Cu") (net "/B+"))
 (segment (start 139.5 41.615) (end 139.27 41.385) (width 0.2) (layer "F.Cu") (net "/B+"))
 (segment (start 141.5 41.695) (end 141.81 41.385) (width 0.2) (layer "F.Cu") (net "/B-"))
 (segment (start 141.5 45.05) (end 141.5 41.695) (width 0.2) (layer "F.Cu") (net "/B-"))
 (segment (start 140.3 69.3) (end 136.875 69.3) (width 0.2) (layer "F.Cu") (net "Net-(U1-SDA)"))
 (segment (start 136.875 69.3) (end 136 70.175) (width 0.2) (layer "F.Cu") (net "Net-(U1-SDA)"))
 (segment (start 133.555 70.175) (end 125.8 62.42) (width 0.2) (layer "F.Cu") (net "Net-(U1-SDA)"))
 (segment (start 136 70.175) (end 133.555 70.175) (width 0.2) (layer "F.Cu") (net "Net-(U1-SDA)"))
 (segment (start 132.22 78.5) (end 145 78.5) (width 0.2) (layer "F.Cu") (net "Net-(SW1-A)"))
 (segment (start 130.265256 49.5) (end 131 49.5) (width 0.2) (layer "F.Cu") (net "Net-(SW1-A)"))
 (segment (start 145 39) (end 144.5 39.5) (width 0.2) (layer "F.Cu") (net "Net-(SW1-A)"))
 (segment (start 131 46.9) (end 132.15 45.75) (width 0.2) (layer "F.Cu") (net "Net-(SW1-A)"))
 (segment (start 126.5 72.78) (end 132.22 78.5) (width 0.2) (layer "F.Cu") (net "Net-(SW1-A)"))
 (segment (start 128.75 47.984744) (end 130.265256 49.5) (width 0.2) (layer "F.Cu") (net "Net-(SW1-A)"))
 (segment (start 128.75 40.75) (end 128.75 47.984744) (width 0.2) (layer "F.Cu") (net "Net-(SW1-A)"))
 (segment (start 131 49.5) (end 131 46.9) (width 0.2) (layer "F.Cu") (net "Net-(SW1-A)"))
 (segment (start 144.5 39.5) (end 130 39.5) (width 0.2) (layer "F.Cu") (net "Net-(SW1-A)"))
 (segment (start 130 39.5) (end 128.75 40.75) (width 0.2) (layer "F.Cu") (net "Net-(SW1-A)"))
 (segment (start 145 78.5) (end 145 39) (width 0.2) (layer "F.Cu") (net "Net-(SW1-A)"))
 (segment (start 140.4125 64.5) (end 140.8 64.8875) (width 0.2) (layer "F.Cu") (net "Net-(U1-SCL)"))
 (segment (start 126.3 59.88) (end 131.92 65.5) (width 0.2) (layer "F.Cu") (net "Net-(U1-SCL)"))
 (segment (start 125.8 59.88) (end 126.3 59.88) (width 0.2) (layer "F.Cu") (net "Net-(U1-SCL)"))
 (segment (start 140.8 64.8875) (end 140.8 69.3) (width 0.2) (layer "F.Cu") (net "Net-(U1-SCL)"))
 (segment (start 131.92 65.5) (end 139.4125 65.5) (width 0.2) (layer "F.Cu") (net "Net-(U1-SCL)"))
 (segment (start 139.4125 65.5) (end 140.4125 64.5) (width 0.2) (layer "F.Cu") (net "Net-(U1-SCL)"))
 (segment (start 134.19 41.385) (end 130.0375 45.5375) (width 0.2) (layer "F.Cu") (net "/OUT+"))
 (segment (start 130.0375 45.5375) (end 129.85 45.725) (width 0.2) (layer "F.Cu") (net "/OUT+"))
 (segment (start 129.15 45.525) (end 129.15 47.3) (width 0.2) (layer "F.Cu") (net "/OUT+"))
 (segment (start 129.15 45.525) (end 130.025 45.525) (width 0.2) (layer "F.Cu") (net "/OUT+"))
 (segment (start 130.025 45.525) (end 130.0375 45.5375) (width 0.2) (layer "F.Cu") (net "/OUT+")))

